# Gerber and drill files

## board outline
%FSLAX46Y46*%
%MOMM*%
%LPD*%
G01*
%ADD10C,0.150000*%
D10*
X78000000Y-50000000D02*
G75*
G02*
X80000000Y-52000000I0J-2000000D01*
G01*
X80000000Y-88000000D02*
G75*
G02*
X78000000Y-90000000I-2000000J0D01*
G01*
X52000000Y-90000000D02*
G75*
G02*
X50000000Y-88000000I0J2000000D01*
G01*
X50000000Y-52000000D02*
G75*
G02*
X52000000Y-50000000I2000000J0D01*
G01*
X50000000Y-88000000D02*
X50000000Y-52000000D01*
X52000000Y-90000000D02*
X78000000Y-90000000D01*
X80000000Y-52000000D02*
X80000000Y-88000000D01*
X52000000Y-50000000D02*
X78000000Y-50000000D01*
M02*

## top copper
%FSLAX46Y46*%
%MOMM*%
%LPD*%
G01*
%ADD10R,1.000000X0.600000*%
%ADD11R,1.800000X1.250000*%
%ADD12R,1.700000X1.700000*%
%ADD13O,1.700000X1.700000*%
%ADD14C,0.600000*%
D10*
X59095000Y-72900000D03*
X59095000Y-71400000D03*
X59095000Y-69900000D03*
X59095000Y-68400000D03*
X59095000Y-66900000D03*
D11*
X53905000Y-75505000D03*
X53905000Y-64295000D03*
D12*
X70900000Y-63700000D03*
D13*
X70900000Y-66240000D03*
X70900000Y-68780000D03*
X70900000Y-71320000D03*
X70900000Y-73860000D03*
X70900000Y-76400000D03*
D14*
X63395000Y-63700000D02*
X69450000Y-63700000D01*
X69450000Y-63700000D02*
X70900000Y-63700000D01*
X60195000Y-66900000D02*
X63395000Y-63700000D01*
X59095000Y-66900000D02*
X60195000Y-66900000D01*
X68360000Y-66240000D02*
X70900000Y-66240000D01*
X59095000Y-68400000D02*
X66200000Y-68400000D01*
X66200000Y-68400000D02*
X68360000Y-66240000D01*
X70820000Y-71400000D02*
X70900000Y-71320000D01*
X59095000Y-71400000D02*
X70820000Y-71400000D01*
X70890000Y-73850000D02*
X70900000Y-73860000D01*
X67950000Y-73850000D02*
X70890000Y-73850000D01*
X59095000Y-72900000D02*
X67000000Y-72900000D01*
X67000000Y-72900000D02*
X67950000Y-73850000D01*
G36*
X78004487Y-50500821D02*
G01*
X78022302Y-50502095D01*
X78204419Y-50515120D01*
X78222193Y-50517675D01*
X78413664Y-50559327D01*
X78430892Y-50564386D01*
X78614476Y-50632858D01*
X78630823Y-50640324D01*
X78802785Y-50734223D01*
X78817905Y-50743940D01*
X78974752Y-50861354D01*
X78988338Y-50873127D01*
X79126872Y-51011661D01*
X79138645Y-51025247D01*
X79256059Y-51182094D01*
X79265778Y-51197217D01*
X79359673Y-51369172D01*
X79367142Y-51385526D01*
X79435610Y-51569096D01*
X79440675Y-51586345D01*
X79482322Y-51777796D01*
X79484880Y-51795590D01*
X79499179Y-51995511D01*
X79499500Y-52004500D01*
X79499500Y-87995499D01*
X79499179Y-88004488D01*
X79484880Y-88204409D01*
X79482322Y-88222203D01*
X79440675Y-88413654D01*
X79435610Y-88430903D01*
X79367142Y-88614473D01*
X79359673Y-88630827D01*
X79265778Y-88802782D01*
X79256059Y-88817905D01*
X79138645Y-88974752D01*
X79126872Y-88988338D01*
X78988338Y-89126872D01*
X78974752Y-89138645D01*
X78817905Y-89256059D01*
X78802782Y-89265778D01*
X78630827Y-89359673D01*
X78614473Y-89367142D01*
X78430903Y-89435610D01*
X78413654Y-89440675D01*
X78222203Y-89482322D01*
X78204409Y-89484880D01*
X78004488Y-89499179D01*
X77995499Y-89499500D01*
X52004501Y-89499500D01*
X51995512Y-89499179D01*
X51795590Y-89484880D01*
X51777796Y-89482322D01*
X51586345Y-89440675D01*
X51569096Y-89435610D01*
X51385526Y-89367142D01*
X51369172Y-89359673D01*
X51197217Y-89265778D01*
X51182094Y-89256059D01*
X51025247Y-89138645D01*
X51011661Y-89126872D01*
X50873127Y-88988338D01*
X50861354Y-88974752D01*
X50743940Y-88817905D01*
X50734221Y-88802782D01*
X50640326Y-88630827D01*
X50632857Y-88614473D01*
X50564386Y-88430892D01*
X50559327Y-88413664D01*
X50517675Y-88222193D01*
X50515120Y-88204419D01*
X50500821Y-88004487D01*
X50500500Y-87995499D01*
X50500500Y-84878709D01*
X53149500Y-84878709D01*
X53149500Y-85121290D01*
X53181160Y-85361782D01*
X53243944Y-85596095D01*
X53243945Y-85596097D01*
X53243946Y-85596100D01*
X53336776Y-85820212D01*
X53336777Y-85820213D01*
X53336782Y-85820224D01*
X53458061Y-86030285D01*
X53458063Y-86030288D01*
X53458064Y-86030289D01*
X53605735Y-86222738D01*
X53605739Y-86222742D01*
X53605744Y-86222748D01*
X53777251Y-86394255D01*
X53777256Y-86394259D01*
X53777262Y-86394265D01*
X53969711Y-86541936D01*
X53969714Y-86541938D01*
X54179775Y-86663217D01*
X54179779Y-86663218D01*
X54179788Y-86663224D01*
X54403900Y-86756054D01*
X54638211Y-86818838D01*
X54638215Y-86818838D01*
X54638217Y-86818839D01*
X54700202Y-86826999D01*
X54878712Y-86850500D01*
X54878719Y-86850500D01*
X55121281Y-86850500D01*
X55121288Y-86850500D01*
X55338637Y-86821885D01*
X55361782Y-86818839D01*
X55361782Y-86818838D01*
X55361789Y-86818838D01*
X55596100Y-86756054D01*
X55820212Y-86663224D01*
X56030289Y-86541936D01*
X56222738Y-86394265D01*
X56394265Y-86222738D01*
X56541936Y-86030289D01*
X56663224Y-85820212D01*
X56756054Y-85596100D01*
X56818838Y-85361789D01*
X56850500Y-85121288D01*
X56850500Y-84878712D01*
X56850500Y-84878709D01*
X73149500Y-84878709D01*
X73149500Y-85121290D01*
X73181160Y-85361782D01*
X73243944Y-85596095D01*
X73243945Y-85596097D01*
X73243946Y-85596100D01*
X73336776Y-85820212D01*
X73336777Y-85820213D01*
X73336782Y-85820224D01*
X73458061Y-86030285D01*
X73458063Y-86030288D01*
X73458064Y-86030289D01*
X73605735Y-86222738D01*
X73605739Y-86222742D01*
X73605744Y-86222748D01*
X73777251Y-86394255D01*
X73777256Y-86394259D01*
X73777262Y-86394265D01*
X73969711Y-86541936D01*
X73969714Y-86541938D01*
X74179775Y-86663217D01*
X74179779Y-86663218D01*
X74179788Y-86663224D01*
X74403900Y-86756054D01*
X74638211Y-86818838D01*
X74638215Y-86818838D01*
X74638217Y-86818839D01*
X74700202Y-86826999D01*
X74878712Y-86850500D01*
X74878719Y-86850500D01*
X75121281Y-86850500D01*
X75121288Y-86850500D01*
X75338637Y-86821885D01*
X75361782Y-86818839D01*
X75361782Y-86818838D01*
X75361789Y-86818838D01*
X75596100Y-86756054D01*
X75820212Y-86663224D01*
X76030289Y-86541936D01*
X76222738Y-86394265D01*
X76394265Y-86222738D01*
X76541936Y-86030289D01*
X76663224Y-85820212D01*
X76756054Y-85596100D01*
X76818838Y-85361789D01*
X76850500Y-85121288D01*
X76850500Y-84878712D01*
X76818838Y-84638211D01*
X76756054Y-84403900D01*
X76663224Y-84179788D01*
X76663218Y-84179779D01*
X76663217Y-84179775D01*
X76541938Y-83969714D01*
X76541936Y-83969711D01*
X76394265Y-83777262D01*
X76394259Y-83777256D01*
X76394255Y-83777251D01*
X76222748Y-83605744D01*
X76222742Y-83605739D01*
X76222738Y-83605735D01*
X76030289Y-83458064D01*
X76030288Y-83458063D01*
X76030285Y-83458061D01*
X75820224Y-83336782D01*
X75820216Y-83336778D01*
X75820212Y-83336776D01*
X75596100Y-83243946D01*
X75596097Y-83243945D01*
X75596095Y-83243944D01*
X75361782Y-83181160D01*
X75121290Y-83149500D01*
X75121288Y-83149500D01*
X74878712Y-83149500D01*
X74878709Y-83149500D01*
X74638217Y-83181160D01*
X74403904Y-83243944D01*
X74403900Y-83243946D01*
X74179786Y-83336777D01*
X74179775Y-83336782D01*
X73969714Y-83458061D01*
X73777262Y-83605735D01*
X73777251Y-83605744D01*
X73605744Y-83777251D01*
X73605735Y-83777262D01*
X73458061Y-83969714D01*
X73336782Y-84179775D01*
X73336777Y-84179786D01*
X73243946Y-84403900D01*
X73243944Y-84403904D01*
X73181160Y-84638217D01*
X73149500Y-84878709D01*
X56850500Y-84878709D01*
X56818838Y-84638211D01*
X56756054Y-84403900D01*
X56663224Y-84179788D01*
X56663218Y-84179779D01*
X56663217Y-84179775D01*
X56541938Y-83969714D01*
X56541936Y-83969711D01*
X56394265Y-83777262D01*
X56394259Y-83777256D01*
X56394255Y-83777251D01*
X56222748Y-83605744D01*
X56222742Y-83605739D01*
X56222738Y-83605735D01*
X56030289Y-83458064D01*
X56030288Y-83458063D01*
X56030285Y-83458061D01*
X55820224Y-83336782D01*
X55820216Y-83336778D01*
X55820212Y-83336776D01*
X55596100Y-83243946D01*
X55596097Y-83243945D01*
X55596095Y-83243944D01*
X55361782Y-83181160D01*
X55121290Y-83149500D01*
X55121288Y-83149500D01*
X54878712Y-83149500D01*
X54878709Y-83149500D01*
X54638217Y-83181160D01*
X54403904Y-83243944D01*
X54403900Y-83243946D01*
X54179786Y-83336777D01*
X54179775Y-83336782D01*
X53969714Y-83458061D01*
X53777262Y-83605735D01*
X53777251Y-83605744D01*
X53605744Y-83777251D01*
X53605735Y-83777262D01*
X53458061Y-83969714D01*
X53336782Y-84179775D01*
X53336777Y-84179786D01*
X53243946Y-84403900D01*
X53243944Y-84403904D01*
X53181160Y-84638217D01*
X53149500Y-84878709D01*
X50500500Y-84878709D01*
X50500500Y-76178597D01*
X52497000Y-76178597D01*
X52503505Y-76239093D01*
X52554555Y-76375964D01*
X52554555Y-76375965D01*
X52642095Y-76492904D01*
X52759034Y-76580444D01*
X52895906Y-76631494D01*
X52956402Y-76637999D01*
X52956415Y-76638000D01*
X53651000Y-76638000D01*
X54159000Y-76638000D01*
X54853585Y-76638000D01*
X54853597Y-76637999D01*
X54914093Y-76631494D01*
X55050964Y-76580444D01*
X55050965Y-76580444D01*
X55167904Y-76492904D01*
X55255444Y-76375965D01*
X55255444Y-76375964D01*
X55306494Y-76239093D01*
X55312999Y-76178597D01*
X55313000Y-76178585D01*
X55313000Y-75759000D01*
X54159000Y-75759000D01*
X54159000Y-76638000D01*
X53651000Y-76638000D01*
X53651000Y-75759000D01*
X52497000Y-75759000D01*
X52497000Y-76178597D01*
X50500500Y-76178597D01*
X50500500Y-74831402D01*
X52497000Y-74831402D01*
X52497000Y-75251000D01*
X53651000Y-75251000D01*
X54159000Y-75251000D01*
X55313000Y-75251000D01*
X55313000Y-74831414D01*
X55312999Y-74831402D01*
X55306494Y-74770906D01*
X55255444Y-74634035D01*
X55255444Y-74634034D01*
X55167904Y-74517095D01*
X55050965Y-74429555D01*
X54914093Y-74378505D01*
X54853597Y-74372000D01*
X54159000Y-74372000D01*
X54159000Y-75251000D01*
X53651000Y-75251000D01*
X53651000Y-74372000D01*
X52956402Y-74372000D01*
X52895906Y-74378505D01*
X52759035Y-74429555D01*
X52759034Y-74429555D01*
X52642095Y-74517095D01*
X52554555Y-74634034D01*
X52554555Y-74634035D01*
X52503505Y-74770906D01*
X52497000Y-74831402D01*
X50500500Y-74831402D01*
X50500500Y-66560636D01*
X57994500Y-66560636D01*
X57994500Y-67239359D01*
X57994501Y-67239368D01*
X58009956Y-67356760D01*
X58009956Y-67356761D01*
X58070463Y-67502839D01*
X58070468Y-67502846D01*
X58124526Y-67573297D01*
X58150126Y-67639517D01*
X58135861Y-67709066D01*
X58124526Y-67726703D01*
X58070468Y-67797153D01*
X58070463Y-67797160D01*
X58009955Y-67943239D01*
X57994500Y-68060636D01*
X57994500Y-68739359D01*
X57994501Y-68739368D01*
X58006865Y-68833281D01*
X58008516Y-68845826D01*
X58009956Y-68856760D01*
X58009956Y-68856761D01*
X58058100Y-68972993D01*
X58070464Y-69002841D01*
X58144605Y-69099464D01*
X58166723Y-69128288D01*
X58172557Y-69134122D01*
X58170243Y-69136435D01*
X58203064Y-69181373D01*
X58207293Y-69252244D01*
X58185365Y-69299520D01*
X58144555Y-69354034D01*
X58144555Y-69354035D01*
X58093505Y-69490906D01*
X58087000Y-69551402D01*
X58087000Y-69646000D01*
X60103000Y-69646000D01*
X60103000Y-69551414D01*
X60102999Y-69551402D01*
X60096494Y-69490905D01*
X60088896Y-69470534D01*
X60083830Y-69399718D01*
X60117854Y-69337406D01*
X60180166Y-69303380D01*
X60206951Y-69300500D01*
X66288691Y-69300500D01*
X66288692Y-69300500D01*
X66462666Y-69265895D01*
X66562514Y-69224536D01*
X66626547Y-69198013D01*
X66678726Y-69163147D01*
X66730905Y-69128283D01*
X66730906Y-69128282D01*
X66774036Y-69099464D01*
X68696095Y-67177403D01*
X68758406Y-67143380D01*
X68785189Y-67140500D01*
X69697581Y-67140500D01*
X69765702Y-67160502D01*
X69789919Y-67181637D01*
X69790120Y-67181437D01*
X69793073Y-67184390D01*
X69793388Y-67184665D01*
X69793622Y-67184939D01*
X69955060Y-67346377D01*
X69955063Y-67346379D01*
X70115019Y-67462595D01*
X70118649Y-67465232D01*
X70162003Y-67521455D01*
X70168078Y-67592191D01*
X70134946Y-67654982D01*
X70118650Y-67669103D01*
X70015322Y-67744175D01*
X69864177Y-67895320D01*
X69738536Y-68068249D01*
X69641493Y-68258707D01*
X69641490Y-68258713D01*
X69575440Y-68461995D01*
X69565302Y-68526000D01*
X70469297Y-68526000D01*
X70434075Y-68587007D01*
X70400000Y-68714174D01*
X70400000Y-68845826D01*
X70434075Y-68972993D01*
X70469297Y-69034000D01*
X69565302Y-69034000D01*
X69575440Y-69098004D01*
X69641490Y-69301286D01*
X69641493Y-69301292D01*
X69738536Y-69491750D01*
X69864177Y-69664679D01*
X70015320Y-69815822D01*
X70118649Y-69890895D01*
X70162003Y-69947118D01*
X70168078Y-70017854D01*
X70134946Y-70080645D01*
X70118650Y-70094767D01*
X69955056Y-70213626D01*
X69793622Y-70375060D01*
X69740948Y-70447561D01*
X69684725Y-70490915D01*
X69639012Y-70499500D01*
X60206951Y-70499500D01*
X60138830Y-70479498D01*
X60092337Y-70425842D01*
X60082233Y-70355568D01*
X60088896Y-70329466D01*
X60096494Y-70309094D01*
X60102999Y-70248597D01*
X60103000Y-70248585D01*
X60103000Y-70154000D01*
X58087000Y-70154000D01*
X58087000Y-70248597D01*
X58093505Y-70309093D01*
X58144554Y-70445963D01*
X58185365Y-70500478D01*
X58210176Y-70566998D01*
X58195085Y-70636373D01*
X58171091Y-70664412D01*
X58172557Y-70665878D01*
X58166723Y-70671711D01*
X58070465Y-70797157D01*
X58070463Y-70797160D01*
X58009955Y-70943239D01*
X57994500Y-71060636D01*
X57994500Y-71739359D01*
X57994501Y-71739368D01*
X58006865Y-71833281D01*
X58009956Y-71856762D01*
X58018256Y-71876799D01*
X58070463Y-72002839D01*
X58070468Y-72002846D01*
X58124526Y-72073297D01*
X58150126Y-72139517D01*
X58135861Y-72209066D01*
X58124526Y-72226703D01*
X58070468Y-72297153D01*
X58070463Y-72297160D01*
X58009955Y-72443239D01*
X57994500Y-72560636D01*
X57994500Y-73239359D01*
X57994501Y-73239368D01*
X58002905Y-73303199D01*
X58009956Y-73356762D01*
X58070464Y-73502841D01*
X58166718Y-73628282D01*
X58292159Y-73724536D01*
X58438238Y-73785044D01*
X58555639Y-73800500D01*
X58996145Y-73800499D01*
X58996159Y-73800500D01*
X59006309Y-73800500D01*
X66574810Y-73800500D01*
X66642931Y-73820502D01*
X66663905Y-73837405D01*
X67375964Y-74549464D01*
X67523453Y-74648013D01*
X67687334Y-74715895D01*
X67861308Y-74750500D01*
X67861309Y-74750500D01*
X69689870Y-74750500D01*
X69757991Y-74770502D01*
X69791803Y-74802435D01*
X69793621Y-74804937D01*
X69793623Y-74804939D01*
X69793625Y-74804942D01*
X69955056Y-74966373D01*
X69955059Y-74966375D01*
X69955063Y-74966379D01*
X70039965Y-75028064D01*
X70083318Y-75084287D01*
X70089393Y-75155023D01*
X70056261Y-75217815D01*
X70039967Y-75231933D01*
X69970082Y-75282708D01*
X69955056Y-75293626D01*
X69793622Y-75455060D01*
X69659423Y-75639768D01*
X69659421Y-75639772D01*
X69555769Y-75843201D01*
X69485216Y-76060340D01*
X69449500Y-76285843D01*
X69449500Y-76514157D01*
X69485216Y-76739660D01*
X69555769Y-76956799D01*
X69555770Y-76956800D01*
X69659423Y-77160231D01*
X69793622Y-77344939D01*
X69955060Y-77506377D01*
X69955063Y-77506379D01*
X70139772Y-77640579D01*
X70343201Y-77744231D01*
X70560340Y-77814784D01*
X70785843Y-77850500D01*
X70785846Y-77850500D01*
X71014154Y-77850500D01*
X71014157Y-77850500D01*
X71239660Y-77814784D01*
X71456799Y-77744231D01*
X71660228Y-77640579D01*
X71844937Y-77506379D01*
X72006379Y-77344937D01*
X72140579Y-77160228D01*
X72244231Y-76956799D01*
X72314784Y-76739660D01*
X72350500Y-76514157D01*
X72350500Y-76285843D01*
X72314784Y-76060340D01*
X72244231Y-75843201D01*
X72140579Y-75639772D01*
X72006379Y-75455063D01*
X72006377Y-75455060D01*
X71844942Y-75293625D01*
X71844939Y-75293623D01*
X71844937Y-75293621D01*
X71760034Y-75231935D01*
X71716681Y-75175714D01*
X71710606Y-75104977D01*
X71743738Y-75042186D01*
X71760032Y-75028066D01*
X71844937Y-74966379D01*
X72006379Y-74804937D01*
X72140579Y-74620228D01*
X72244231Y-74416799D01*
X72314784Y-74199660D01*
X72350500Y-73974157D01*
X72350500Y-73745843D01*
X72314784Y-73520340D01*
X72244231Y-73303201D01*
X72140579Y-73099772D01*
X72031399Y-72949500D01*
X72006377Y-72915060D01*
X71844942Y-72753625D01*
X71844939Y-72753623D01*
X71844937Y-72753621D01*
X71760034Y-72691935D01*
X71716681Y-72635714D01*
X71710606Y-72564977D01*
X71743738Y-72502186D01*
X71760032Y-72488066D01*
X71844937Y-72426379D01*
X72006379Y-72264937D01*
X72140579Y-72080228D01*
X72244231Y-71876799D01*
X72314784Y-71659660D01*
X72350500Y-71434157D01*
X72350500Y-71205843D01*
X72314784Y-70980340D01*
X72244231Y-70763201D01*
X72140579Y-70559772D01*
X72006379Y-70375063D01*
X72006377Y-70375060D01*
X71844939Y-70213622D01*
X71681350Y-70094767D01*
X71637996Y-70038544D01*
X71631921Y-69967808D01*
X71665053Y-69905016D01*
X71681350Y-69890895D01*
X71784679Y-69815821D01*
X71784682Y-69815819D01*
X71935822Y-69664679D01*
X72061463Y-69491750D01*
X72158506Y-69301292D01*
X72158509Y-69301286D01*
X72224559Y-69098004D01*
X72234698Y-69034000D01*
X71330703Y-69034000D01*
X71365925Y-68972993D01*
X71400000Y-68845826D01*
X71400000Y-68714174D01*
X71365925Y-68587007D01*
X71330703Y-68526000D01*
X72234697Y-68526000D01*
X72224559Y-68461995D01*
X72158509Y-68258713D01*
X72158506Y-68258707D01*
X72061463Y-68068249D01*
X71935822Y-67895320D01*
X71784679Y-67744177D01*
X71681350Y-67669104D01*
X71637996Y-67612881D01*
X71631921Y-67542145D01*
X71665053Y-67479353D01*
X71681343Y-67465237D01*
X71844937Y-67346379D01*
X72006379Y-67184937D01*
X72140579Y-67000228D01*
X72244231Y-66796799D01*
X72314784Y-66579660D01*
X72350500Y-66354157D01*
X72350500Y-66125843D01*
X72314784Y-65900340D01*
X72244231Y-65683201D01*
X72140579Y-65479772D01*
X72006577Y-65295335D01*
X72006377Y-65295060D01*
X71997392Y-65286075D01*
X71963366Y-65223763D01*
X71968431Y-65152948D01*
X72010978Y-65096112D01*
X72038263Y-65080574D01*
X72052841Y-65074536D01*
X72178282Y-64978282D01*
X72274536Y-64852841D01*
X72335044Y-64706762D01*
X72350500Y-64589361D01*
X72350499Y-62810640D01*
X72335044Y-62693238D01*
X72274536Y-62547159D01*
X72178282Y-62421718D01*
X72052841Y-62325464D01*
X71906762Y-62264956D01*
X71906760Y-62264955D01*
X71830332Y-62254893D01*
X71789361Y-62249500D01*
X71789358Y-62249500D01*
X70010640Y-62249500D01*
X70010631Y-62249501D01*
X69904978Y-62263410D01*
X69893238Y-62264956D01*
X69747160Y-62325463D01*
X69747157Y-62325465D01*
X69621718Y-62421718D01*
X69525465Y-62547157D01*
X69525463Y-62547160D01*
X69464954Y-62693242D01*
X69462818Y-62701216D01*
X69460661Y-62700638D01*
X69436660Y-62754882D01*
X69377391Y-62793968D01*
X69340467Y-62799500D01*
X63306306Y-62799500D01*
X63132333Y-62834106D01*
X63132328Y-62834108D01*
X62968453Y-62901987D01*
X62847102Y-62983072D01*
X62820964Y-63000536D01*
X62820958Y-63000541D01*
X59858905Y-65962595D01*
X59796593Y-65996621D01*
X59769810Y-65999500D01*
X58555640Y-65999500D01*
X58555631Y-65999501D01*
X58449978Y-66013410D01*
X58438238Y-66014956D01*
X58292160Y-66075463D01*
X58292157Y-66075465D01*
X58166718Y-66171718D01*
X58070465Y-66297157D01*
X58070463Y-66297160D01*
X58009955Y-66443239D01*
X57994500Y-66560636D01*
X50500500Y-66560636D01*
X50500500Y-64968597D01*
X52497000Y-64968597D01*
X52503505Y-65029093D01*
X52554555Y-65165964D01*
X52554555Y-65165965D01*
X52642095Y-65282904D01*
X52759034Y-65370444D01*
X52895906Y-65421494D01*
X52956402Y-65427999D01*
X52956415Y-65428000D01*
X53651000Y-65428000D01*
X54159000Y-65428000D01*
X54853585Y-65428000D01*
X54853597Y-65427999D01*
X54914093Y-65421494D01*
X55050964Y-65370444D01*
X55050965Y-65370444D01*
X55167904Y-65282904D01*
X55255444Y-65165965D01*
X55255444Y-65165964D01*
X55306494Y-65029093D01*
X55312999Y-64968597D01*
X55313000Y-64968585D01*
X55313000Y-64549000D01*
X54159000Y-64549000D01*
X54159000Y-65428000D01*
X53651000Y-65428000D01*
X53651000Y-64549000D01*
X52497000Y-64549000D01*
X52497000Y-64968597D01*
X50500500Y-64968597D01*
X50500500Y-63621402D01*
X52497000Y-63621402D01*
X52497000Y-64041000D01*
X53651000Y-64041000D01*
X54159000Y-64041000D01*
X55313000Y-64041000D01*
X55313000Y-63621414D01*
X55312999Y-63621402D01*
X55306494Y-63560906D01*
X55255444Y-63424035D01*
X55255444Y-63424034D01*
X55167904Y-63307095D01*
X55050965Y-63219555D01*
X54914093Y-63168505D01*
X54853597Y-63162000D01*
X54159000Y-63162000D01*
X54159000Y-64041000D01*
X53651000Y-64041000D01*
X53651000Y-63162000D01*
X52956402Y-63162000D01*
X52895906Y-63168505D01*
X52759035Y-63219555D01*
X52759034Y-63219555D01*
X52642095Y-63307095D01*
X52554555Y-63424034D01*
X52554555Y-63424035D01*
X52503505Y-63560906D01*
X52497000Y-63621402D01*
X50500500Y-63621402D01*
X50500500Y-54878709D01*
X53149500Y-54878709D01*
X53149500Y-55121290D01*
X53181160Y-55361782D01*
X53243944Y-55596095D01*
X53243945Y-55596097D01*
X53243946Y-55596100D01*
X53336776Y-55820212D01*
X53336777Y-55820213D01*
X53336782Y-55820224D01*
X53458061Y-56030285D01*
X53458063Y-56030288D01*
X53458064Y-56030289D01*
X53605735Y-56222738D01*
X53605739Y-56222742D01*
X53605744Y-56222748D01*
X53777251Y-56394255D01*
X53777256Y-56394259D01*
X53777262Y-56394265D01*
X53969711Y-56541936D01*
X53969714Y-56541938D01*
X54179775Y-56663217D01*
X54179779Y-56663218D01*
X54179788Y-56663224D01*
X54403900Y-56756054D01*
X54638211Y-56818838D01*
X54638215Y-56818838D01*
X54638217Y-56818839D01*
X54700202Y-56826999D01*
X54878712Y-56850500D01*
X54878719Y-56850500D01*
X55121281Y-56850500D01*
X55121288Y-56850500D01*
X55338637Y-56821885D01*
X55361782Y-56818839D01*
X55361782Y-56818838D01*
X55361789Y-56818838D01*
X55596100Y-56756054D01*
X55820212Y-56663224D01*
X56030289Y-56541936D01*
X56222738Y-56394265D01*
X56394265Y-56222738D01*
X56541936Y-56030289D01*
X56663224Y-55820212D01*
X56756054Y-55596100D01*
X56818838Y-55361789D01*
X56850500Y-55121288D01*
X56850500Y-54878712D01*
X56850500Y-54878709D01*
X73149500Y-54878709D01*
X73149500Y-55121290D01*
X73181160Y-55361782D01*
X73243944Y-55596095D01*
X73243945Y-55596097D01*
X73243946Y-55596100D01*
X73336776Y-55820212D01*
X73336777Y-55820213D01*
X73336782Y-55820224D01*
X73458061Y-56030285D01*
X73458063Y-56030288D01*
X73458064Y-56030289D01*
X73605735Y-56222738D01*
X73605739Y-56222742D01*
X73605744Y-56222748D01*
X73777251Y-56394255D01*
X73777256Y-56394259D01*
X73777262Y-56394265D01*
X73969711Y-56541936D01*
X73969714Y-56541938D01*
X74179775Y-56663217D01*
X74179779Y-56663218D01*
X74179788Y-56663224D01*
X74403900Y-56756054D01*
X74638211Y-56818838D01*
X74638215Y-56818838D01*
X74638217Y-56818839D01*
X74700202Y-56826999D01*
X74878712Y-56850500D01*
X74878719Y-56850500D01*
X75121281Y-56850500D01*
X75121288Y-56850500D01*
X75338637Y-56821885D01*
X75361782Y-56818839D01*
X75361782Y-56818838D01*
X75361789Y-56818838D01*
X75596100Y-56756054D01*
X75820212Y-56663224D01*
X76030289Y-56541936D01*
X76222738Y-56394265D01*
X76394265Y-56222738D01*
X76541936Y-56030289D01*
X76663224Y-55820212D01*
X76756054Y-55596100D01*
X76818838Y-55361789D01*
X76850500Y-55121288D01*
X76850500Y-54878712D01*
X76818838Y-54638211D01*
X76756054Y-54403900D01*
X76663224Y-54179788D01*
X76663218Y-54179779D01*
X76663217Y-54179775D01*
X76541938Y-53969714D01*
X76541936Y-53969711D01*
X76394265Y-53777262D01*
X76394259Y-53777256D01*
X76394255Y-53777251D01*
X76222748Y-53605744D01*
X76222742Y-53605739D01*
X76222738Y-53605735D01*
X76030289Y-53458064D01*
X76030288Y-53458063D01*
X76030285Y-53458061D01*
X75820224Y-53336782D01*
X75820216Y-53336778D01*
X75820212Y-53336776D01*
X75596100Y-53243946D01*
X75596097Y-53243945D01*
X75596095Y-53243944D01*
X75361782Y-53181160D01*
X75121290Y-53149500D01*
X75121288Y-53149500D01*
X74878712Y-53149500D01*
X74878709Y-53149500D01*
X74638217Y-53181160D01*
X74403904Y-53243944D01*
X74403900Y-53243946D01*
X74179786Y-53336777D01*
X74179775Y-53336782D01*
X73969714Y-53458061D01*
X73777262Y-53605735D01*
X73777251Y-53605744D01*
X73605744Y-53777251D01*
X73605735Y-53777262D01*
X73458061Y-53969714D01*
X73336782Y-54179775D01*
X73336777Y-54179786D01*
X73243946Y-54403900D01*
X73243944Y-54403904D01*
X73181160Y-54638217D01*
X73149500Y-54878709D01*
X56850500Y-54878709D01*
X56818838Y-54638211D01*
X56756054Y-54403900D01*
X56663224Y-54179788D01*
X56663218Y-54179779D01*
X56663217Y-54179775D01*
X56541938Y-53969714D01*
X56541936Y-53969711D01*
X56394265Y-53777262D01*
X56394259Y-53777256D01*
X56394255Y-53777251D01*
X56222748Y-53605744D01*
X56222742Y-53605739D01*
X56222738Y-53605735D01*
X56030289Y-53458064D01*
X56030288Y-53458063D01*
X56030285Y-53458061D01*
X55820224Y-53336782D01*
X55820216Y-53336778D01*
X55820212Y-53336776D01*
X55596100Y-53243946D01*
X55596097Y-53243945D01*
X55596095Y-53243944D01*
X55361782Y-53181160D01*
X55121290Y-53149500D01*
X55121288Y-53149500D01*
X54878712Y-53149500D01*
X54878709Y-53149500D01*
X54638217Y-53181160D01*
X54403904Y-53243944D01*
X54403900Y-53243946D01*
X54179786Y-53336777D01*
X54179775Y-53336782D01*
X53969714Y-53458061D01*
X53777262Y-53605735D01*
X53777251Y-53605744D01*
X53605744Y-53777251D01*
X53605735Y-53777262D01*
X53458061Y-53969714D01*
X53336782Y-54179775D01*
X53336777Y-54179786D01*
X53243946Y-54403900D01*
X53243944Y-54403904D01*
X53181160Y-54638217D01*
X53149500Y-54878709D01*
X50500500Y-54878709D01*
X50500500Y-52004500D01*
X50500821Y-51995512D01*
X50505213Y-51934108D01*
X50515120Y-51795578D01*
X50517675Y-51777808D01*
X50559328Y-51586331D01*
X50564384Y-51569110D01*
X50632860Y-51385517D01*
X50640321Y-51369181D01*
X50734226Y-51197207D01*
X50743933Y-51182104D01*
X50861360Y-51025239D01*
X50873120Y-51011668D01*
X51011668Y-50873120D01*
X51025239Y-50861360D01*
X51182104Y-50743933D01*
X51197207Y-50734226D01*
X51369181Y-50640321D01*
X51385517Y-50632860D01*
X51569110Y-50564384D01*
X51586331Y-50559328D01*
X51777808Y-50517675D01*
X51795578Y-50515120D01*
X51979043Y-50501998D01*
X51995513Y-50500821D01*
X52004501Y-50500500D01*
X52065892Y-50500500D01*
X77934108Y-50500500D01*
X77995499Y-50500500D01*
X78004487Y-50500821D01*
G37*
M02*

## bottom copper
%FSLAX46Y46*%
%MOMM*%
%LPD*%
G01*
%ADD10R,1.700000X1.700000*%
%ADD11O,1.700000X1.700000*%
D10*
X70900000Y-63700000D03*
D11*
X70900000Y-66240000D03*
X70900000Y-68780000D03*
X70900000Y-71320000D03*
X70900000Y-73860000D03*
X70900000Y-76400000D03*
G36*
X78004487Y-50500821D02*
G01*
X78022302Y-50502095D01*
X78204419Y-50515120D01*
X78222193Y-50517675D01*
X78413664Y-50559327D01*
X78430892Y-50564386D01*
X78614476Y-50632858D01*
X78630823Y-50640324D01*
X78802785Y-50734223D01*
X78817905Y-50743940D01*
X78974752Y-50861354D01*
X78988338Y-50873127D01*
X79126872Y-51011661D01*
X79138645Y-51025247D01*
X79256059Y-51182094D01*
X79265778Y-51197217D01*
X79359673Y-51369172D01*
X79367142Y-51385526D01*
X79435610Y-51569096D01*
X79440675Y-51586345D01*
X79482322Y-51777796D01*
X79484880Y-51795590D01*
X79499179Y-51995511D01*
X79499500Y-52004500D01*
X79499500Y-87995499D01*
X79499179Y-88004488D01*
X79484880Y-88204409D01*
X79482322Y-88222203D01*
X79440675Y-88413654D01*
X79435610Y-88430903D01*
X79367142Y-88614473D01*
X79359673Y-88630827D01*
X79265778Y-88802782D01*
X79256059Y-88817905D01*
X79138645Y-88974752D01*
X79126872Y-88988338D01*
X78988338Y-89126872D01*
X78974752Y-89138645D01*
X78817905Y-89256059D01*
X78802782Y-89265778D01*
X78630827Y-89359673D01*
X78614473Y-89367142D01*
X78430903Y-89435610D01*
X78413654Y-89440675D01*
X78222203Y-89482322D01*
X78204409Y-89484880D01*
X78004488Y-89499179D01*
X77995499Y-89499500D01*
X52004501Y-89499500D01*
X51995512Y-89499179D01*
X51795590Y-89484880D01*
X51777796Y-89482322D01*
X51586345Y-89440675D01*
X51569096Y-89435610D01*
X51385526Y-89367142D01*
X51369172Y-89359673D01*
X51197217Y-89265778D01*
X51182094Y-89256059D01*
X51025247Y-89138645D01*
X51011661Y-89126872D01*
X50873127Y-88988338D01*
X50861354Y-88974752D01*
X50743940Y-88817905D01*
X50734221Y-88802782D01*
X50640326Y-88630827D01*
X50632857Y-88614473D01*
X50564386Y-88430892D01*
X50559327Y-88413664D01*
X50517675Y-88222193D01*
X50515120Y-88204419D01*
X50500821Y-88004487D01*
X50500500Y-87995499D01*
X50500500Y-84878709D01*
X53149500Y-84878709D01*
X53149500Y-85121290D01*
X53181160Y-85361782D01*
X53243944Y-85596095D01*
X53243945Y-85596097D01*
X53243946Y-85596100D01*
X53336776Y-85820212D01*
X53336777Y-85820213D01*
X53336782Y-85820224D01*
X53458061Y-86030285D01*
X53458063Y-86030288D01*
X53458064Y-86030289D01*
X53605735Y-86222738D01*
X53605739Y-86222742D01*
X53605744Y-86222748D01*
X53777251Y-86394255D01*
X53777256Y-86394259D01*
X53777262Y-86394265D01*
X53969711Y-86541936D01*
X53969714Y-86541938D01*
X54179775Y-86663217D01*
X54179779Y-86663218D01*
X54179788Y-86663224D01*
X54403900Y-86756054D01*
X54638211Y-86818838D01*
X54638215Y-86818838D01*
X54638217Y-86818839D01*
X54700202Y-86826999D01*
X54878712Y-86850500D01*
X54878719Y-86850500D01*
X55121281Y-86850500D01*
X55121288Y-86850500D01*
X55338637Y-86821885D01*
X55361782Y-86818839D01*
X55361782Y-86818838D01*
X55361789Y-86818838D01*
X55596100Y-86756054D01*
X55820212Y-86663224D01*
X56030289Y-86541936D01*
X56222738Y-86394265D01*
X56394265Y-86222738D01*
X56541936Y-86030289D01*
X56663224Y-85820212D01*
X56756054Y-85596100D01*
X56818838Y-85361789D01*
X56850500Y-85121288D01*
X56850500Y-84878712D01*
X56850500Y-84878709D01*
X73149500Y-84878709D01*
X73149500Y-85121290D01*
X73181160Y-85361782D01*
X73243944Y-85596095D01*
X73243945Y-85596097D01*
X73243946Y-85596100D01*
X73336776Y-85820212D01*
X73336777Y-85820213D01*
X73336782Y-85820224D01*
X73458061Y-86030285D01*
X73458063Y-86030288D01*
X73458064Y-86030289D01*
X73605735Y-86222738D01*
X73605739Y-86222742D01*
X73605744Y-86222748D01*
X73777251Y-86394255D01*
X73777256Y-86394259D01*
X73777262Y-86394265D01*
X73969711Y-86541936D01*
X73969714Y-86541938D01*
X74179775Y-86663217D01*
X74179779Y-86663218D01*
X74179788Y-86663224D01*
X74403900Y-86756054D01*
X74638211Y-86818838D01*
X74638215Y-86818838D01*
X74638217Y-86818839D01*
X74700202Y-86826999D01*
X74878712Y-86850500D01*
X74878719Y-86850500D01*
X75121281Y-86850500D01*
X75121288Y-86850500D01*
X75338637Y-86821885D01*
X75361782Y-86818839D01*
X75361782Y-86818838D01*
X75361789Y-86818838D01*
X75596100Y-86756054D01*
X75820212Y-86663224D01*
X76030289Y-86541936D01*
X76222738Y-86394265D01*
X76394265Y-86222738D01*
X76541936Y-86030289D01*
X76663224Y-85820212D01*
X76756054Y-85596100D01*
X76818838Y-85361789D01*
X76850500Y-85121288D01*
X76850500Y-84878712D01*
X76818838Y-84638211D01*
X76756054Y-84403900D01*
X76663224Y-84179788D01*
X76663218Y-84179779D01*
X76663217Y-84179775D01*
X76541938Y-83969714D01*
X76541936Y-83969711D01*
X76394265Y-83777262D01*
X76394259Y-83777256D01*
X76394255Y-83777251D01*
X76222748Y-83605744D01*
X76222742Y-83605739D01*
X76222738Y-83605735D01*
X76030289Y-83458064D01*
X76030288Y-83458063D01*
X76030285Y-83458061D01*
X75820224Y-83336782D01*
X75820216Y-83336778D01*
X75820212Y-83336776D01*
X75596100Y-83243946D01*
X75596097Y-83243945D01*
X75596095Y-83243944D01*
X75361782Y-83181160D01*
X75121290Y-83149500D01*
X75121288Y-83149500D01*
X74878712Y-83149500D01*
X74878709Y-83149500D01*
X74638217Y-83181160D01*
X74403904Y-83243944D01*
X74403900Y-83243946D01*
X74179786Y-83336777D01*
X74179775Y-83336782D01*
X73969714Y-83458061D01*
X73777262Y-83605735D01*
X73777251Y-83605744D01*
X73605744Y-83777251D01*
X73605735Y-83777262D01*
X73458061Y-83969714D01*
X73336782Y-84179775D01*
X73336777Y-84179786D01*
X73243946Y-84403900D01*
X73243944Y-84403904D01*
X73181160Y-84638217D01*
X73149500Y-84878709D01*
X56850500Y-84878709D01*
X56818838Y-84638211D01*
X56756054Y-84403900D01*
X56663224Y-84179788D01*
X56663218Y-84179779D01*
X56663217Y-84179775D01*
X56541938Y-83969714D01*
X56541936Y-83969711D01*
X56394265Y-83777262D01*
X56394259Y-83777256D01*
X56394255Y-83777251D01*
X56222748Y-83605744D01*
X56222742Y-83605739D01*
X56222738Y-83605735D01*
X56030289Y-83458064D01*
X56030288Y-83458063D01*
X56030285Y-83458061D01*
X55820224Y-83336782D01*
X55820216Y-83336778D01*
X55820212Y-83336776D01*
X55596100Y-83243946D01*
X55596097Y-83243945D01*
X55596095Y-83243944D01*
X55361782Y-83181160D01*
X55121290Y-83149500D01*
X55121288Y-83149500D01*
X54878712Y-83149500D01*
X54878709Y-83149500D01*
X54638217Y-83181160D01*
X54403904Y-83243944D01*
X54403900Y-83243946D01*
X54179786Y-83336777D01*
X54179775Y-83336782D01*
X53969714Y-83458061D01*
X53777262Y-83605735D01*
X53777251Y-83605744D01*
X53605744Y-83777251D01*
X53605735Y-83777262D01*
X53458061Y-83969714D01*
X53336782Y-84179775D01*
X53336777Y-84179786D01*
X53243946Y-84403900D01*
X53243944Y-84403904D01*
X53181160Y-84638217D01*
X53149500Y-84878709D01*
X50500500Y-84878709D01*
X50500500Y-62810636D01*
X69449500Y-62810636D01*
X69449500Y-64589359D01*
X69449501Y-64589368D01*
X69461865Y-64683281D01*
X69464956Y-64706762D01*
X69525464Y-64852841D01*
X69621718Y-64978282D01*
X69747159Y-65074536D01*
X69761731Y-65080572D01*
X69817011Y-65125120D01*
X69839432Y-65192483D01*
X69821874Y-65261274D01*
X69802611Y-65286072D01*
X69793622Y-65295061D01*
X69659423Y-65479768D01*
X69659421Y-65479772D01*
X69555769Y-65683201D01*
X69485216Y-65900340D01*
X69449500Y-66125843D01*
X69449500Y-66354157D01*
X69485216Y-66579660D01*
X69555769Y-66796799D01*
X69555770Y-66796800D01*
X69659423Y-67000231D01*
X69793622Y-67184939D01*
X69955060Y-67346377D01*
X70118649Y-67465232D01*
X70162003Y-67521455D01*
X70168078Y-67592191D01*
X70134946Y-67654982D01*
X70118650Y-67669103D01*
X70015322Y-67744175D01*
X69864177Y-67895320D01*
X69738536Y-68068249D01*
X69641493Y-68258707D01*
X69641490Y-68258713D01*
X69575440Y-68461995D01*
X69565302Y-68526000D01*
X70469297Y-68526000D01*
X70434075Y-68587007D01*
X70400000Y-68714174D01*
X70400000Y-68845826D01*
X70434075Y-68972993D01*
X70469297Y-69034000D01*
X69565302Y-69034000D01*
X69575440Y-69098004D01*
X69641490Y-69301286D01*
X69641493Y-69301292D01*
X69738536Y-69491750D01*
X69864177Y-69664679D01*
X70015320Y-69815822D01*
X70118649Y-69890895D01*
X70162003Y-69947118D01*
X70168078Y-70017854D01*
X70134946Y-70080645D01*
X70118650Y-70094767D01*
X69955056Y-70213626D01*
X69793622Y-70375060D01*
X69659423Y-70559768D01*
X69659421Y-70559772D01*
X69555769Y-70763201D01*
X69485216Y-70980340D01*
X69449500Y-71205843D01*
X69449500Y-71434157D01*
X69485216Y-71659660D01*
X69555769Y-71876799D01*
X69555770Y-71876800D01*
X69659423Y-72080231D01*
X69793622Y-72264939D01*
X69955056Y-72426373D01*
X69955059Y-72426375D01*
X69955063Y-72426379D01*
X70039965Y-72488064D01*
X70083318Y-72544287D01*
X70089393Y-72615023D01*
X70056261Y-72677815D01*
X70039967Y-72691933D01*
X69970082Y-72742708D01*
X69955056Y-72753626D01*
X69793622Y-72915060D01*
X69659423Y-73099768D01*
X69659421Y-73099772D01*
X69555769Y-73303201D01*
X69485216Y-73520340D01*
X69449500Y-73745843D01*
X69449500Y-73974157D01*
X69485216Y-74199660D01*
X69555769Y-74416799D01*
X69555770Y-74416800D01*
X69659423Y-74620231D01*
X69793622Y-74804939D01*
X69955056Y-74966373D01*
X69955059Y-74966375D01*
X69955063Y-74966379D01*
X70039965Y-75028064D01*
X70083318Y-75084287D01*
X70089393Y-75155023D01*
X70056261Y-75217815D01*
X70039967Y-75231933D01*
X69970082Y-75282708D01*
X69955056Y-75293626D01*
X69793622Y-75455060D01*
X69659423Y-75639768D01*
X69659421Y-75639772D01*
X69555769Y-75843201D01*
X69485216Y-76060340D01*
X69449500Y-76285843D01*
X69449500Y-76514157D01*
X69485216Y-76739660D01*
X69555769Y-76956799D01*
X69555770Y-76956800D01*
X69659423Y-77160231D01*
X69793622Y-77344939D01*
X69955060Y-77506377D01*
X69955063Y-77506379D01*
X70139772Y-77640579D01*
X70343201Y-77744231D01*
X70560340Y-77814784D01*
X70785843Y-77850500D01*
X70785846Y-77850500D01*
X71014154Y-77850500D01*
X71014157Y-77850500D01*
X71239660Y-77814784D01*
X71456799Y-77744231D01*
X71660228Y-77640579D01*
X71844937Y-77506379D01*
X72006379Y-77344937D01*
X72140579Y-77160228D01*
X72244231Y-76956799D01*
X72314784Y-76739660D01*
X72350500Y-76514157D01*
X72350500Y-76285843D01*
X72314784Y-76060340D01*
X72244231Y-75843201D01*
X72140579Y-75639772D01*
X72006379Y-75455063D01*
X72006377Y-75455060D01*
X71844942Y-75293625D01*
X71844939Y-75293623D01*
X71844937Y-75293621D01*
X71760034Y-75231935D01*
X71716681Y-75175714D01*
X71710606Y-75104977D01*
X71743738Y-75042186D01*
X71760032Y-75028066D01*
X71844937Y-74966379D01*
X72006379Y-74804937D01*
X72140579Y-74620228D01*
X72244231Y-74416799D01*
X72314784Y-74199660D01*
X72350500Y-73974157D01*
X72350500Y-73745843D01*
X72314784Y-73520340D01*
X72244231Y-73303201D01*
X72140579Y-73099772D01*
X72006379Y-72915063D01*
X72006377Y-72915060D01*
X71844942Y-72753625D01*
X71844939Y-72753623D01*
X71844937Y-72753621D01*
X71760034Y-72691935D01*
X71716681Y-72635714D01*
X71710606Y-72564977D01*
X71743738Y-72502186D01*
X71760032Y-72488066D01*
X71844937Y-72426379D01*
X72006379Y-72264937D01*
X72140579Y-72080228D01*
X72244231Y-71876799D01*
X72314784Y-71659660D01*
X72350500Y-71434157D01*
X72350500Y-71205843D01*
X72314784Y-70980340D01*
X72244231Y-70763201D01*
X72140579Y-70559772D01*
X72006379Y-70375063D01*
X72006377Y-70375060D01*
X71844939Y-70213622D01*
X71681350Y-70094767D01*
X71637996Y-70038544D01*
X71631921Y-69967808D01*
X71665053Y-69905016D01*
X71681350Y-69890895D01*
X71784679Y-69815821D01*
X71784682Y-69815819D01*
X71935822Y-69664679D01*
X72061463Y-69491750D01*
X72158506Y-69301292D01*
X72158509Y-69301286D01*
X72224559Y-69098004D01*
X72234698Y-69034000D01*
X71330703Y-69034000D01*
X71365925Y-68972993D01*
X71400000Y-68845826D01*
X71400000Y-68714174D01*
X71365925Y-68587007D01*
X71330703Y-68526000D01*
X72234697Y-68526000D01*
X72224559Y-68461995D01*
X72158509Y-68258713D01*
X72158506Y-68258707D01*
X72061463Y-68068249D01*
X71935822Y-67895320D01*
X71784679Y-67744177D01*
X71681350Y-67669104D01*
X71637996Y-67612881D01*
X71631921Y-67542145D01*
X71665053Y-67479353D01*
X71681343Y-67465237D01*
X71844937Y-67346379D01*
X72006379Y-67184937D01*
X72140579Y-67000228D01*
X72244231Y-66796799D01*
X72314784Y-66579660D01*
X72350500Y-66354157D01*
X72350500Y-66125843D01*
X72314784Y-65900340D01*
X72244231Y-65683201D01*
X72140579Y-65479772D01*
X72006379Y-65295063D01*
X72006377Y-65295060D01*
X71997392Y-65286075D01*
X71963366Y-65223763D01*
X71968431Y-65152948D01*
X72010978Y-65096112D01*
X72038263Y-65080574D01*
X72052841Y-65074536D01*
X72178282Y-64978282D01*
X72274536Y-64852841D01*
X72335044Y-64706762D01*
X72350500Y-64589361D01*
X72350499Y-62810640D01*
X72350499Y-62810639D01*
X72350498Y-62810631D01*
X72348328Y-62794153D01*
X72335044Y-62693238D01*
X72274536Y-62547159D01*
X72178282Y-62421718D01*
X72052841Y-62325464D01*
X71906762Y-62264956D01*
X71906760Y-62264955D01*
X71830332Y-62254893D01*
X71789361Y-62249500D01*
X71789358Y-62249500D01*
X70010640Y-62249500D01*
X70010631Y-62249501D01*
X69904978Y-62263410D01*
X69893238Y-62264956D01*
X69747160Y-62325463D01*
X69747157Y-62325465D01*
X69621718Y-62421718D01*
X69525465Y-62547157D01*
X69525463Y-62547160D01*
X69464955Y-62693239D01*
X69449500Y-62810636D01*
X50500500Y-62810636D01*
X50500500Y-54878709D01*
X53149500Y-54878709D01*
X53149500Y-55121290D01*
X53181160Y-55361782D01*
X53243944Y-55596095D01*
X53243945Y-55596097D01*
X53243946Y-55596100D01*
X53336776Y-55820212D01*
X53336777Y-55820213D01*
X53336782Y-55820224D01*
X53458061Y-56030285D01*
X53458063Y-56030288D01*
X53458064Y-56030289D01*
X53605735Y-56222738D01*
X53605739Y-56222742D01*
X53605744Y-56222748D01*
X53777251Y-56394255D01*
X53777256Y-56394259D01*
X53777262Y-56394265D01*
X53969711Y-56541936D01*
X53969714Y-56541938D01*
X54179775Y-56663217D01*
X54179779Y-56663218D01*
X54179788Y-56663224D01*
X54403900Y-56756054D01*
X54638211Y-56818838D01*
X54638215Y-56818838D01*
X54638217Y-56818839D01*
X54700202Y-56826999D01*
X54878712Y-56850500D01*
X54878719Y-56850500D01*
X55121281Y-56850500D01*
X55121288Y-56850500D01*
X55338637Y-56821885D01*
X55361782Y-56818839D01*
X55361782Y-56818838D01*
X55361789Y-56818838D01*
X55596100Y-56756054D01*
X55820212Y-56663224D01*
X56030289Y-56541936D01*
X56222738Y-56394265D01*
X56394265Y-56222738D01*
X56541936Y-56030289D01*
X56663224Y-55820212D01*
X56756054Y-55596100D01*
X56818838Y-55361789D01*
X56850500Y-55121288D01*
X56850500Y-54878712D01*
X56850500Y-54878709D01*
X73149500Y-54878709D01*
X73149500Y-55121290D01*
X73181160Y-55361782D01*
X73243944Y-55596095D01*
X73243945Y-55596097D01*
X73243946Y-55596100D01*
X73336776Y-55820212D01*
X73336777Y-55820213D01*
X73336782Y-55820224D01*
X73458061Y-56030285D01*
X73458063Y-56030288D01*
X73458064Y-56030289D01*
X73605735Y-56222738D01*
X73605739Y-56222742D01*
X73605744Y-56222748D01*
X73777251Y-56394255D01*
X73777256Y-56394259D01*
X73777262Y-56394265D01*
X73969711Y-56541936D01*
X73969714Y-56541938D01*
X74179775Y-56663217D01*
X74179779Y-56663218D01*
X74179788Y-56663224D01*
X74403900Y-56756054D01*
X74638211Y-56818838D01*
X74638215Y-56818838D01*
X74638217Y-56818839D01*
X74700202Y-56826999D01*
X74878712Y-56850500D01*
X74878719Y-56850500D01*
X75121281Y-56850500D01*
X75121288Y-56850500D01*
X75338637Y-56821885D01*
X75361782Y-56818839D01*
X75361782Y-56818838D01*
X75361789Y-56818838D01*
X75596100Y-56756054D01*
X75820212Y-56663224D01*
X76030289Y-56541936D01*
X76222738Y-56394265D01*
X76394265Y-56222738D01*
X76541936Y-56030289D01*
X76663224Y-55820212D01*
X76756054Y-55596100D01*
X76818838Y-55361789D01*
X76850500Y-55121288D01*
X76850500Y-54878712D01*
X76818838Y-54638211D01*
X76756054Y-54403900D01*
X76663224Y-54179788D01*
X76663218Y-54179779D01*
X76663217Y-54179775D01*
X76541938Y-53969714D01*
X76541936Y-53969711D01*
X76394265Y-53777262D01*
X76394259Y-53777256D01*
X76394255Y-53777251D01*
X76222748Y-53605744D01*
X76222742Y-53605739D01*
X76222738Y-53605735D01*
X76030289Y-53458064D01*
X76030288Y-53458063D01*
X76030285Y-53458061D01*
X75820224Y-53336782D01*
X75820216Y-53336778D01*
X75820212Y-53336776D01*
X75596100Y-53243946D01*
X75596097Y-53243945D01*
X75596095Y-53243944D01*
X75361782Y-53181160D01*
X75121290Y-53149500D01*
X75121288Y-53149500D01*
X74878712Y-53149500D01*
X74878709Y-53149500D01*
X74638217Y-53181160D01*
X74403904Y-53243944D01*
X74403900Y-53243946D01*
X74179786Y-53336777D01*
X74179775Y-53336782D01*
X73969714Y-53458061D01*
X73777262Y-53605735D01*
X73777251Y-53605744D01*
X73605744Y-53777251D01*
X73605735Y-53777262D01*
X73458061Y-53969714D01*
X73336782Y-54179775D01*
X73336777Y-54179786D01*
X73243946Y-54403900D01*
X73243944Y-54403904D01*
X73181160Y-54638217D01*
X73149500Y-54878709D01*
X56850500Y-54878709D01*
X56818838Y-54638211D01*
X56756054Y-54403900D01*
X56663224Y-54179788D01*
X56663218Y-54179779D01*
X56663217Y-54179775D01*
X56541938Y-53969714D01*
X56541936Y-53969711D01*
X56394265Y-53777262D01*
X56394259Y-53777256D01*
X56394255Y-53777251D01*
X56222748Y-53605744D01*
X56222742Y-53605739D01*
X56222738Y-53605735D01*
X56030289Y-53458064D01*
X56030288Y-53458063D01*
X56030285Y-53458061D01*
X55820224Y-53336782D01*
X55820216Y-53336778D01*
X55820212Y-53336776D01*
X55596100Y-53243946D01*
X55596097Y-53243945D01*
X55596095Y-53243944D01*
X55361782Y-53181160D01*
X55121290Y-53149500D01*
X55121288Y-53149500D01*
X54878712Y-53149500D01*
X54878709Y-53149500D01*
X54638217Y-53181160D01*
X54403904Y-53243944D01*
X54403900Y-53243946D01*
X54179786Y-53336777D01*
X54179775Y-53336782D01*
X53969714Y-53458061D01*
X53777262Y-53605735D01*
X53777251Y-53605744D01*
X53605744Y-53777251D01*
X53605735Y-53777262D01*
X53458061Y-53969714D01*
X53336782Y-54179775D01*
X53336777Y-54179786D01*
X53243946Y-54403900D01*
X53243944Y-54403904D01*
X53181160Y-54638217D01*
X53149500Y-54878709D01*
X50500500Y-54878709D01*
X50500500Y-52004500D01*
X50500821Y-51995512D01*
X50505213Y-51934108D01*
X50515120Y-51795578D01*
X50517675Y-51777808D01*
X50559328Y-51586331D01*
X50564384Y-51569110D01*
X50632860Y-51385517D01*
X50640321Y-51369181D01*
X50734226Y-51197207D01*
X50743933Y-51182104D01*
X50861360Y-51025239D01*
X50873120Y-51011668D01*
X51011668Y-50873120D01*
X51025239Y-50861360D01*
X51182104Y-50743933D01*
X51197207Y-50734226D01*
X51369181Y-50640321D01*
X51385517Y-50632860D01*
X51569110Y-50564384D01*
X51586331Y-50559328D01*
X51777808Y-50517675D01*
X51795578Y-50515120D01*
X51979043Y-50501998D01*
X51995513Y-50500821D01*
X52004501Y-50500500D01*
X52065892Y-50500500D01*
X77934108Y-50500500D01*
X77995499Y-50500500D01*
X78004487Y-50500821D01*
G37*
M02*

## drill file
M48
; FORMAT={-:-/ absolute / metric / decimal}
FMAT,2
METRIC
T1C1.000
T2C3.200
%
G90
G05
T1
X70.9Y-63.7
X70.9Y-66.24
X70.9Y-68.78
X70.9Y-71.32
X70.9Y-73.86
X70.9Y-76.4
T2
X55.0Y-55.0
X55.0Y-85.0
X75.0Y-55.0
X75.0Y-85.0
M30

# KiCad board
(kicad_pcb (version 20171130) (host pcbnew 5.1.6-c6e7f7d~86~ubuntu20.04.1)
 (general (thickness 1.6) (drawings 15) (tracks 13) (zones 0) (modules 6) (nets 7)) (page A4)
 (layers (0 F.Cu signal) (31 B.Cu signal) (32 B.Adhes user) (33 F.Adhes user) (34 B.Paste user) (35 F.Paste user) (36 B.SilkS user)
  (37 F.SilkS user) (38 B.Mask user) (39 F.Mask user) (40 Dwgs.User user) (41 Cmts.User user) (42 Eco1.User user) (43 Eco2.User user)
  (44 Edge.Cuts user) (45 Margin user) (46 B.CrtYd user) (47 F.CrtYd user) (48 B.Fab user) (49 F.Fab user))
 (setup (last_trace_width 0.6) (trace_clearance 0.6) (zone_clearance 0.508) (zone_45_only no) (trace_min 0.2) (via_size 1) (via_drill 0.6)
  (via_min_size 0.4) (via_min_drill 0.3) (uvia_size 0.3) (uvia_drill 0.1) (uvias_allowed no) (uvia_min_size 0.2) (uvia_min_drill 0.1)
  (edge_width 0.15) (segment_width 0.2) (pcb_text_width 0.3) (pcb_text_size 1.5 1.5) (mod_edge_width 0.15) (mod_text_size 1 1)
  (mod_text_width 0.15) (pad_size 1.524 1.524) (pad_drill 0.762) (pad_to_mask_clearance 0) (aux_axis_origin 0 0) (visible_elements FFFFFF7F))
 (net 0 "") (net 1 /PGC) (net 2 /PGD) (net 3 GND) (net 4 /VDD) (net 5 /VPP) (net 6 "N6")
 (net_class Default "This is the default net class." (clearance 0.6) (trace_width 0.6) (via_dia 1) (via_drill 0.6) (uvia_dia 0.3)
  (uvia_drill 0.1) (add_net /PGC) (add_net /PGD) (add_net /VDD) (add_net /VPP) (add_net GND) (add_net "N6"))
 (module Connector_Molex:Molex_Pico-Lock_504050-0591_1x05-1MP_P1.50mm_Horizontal (layer F.Cu) (at 56.3 69.9 90)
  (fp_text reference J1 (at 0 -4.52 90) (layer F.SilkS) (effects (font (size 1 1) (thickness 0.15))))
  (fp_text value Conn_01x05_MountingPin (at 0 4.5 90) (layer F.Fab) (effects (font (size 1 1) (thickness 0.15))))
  (pad 1 smd rect (at -3 2.795 90) (size 0.6 1) (layers F.Cu F.Paste F.Mask) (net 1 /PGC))
  (pad 2 smd rect (at -1.5 2.795 90) (size 0.6 1) (layers F.Cu F.Paste F.Mask) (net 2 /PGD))
  (pad 3 smd rect (at 0 2.795 90) (size 0.6 1) (layers F.Cu F.Paste F.Mask) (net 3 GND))
  (pad 4 smd rect (at 1.5 2.795 90) (size 0.6 1) (layers F.Cu F.Paste F.Mask) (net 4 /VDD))
  (pad 5 smd rect (at 3 2.795 90) (size 0.6 1) (layers F.Cu F.Paste F.Mask) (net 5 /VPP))
  (pad MP smd rect (at -5.605 -2.395 90) (size 1.25 1.8) (layers F.Cu F.Paste F.Mask) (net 3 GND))
  (pad MP smd rect (at 5.605 -2.395 90) (size 1.25 1.8) (layers F.Cu F.Paste F.Mask) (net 3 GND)))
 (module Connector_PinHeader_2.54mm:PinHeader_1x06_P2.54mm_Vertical (layer F.Cu) (at 70.9 63.7)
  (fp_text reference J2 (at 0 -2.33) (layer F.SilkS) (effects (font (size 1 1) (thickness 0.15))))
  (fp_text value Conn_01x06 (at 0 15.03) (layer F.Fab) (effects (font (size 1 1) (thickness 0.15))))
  (pad 1 thru_hole rect (at 0 0) (size 1.7 1.7) (drill 1) (layers *.Cu *.Mask) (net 5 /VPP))
  (pad 2 thru_hole oval (at 0 2.54) (size 1.7 1.7) (drill 1) (layers *.Cu *.Mask) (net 4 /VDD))
  (pad 3 thru_hole oval (at 0 5.08) (size 1.7 1.7) (drill 1) (layers *.Cu *.Mask) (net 3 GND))
  (pad 4 thru_hole oval (at 0 7.62) (size 1.7 1.7) (drill 1) (layers *.Cu *.Mask) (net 2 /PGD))
  (pad 5 thru_hole oval (at 0 10.16) (size 1.7 1.7) (drill 1) (layers *.Cu *.Mask) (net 1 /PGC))
  (pad 6 thru_hole oval (at 0 12.7) (size 1.7 1.7) (drill 1) (layers *.Cu *.Mask) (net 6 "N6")))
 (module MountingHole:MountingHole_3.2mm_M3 (layer F.Cu) (at 75 85)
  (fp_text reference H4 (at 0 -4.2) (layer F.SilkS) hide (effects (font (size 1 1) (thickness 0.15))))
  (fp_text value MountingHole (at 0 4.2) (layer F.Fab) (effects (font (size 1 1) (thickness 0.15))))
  (pad 1 np_thru_hole circle (at 0 0) (size 3.2 3.2) (drill 3.2) (layers *.Cu *.Mask)))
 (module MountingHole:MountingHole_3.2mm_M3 (layer F.Cu) (at 55 85)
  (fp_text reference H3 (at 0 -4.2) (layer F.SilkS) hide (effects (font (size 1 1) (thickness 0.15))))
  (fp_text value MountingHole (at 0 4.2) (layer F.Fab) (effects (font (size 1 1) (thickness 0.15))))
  (pad 1 np_thru_hole circle (at 0 0) (size 3.2 3.2) (drill 3.2) (layers *.Cu *.Mask)))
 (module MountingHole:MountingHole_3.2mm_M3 (layer F.Cu) (at 75 55)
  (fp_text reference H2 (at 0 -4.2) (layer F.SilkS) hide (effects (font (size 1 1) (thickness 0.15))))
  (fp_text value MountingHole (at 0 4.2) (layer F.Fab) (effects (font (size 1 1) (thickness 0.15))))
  (pad 1 np_thru_hole circle (at 0 0) (size 3.2 3.2) (drill 3.2) (layers *.Cu *.Mask)))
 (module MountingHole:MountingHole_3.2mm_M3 (layer F.Cu) (at 55 55)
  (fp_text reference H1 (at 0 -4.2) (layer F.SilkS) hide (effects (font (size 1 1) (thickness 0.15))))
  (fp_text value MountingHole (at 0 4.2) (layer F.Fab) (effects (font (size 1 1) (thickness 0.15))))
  (pad 1 np_thru_hole circle (at 0 0) (size 3.2 3.2) (drill 3.2) (layers *.Cu *.Mask)))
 (gr_arc (start 78 52) (end 80 52) (angle -90) (layer Edge.Cuts) (width 0.15))
 (gr_arc (start 78 88) (end 78 90) (angle -90) (layer Edge.Cuts) (width 0.15))
 (gr_arc (start 52 88) (end 50 88) (angle -90) (layer Edge.Cuts) (width 0.15))
 (gr_arc (start 52 52) (end 52 50) (angle -90) (layer Edge.Cuts) (width 0.15))
 (gr_line (start 50 88) (end 50 52) (layer Edge.Cuts) (width 0.15))
 (gr_line (start 52 90) (end 78 90) (layer Edge.Cuts) (width 0.15))
 (gr_line (start 80 52) (end 80 88) (layer Edge.Cuts) (width 0.15))
 (gr_line (start 52 50) (end 78 50) (layer Edge.Cuts) (width 0.15))
 (segment (start 63.395 63.7) (end 69.45 63.7) (width 0.6) (layer F.Cu) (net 5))
 (segment (start 69.45 63.7) (end 70.9 63.7) (width 0.6) (layer F.Cu) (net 5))
 (segment (start 60.195 66.9) (end 63.395 63.7) (width 0.6) (layer F.Cu) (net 5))
 (segment (start 59.095 66.9) (end 60.195 66.9) (width 0.6) (layer F.Cu) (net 5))
 (segment (start 68.36 66.24) (end 70.9 66.24) (width 0.6) (layer F.Cu) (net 4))
 (segment (start 59.095 68.4) (end 66.2 68.4) (width 0.6) (layer F.Cu) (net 4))
 (segment (start 66.2 68.4) (end 68.36 66.24) (width 0.6) (layer F.Cu) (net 4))
 (segment (start 70.82 71.4) (end 70.9 71.32) (width 0.6) (layer F.Cu) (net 2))
 (segment (start 59.095 71.4) (end 70.82 71.4) (width 0.6) (layer F.Cu) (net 2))
 (segment (start 70.89 73.85) (end 70.9 73.86) (width 0.6) (layer F.Cu) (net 1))
 (segment (start 67.95 73.85) (end 70.89 73.85) (width 0.6) (layer F.Cu) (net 1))
 (segment (start 59.095 72.9) (end 67 72.9) (width 0.6) (layer F.Cu) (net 1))
 (segment (start 67 72.9) (end 67.95 73.85) (width 0.6) (layer F.Cu) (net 1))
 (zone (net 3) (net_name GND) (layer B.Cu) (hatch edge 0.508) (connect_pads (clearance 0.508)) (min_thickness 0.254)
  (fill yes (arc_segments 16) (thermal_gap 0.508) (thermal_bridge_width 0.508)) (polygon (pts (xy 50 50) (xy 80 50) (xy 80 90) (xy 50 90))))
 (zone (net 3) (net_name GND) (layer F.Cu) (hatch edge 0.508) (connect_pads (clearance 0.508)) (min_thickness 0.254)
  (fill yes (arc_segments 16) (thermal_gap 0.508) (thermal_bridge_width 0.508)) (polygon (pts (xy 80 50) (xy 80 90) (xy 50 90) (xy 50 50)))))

